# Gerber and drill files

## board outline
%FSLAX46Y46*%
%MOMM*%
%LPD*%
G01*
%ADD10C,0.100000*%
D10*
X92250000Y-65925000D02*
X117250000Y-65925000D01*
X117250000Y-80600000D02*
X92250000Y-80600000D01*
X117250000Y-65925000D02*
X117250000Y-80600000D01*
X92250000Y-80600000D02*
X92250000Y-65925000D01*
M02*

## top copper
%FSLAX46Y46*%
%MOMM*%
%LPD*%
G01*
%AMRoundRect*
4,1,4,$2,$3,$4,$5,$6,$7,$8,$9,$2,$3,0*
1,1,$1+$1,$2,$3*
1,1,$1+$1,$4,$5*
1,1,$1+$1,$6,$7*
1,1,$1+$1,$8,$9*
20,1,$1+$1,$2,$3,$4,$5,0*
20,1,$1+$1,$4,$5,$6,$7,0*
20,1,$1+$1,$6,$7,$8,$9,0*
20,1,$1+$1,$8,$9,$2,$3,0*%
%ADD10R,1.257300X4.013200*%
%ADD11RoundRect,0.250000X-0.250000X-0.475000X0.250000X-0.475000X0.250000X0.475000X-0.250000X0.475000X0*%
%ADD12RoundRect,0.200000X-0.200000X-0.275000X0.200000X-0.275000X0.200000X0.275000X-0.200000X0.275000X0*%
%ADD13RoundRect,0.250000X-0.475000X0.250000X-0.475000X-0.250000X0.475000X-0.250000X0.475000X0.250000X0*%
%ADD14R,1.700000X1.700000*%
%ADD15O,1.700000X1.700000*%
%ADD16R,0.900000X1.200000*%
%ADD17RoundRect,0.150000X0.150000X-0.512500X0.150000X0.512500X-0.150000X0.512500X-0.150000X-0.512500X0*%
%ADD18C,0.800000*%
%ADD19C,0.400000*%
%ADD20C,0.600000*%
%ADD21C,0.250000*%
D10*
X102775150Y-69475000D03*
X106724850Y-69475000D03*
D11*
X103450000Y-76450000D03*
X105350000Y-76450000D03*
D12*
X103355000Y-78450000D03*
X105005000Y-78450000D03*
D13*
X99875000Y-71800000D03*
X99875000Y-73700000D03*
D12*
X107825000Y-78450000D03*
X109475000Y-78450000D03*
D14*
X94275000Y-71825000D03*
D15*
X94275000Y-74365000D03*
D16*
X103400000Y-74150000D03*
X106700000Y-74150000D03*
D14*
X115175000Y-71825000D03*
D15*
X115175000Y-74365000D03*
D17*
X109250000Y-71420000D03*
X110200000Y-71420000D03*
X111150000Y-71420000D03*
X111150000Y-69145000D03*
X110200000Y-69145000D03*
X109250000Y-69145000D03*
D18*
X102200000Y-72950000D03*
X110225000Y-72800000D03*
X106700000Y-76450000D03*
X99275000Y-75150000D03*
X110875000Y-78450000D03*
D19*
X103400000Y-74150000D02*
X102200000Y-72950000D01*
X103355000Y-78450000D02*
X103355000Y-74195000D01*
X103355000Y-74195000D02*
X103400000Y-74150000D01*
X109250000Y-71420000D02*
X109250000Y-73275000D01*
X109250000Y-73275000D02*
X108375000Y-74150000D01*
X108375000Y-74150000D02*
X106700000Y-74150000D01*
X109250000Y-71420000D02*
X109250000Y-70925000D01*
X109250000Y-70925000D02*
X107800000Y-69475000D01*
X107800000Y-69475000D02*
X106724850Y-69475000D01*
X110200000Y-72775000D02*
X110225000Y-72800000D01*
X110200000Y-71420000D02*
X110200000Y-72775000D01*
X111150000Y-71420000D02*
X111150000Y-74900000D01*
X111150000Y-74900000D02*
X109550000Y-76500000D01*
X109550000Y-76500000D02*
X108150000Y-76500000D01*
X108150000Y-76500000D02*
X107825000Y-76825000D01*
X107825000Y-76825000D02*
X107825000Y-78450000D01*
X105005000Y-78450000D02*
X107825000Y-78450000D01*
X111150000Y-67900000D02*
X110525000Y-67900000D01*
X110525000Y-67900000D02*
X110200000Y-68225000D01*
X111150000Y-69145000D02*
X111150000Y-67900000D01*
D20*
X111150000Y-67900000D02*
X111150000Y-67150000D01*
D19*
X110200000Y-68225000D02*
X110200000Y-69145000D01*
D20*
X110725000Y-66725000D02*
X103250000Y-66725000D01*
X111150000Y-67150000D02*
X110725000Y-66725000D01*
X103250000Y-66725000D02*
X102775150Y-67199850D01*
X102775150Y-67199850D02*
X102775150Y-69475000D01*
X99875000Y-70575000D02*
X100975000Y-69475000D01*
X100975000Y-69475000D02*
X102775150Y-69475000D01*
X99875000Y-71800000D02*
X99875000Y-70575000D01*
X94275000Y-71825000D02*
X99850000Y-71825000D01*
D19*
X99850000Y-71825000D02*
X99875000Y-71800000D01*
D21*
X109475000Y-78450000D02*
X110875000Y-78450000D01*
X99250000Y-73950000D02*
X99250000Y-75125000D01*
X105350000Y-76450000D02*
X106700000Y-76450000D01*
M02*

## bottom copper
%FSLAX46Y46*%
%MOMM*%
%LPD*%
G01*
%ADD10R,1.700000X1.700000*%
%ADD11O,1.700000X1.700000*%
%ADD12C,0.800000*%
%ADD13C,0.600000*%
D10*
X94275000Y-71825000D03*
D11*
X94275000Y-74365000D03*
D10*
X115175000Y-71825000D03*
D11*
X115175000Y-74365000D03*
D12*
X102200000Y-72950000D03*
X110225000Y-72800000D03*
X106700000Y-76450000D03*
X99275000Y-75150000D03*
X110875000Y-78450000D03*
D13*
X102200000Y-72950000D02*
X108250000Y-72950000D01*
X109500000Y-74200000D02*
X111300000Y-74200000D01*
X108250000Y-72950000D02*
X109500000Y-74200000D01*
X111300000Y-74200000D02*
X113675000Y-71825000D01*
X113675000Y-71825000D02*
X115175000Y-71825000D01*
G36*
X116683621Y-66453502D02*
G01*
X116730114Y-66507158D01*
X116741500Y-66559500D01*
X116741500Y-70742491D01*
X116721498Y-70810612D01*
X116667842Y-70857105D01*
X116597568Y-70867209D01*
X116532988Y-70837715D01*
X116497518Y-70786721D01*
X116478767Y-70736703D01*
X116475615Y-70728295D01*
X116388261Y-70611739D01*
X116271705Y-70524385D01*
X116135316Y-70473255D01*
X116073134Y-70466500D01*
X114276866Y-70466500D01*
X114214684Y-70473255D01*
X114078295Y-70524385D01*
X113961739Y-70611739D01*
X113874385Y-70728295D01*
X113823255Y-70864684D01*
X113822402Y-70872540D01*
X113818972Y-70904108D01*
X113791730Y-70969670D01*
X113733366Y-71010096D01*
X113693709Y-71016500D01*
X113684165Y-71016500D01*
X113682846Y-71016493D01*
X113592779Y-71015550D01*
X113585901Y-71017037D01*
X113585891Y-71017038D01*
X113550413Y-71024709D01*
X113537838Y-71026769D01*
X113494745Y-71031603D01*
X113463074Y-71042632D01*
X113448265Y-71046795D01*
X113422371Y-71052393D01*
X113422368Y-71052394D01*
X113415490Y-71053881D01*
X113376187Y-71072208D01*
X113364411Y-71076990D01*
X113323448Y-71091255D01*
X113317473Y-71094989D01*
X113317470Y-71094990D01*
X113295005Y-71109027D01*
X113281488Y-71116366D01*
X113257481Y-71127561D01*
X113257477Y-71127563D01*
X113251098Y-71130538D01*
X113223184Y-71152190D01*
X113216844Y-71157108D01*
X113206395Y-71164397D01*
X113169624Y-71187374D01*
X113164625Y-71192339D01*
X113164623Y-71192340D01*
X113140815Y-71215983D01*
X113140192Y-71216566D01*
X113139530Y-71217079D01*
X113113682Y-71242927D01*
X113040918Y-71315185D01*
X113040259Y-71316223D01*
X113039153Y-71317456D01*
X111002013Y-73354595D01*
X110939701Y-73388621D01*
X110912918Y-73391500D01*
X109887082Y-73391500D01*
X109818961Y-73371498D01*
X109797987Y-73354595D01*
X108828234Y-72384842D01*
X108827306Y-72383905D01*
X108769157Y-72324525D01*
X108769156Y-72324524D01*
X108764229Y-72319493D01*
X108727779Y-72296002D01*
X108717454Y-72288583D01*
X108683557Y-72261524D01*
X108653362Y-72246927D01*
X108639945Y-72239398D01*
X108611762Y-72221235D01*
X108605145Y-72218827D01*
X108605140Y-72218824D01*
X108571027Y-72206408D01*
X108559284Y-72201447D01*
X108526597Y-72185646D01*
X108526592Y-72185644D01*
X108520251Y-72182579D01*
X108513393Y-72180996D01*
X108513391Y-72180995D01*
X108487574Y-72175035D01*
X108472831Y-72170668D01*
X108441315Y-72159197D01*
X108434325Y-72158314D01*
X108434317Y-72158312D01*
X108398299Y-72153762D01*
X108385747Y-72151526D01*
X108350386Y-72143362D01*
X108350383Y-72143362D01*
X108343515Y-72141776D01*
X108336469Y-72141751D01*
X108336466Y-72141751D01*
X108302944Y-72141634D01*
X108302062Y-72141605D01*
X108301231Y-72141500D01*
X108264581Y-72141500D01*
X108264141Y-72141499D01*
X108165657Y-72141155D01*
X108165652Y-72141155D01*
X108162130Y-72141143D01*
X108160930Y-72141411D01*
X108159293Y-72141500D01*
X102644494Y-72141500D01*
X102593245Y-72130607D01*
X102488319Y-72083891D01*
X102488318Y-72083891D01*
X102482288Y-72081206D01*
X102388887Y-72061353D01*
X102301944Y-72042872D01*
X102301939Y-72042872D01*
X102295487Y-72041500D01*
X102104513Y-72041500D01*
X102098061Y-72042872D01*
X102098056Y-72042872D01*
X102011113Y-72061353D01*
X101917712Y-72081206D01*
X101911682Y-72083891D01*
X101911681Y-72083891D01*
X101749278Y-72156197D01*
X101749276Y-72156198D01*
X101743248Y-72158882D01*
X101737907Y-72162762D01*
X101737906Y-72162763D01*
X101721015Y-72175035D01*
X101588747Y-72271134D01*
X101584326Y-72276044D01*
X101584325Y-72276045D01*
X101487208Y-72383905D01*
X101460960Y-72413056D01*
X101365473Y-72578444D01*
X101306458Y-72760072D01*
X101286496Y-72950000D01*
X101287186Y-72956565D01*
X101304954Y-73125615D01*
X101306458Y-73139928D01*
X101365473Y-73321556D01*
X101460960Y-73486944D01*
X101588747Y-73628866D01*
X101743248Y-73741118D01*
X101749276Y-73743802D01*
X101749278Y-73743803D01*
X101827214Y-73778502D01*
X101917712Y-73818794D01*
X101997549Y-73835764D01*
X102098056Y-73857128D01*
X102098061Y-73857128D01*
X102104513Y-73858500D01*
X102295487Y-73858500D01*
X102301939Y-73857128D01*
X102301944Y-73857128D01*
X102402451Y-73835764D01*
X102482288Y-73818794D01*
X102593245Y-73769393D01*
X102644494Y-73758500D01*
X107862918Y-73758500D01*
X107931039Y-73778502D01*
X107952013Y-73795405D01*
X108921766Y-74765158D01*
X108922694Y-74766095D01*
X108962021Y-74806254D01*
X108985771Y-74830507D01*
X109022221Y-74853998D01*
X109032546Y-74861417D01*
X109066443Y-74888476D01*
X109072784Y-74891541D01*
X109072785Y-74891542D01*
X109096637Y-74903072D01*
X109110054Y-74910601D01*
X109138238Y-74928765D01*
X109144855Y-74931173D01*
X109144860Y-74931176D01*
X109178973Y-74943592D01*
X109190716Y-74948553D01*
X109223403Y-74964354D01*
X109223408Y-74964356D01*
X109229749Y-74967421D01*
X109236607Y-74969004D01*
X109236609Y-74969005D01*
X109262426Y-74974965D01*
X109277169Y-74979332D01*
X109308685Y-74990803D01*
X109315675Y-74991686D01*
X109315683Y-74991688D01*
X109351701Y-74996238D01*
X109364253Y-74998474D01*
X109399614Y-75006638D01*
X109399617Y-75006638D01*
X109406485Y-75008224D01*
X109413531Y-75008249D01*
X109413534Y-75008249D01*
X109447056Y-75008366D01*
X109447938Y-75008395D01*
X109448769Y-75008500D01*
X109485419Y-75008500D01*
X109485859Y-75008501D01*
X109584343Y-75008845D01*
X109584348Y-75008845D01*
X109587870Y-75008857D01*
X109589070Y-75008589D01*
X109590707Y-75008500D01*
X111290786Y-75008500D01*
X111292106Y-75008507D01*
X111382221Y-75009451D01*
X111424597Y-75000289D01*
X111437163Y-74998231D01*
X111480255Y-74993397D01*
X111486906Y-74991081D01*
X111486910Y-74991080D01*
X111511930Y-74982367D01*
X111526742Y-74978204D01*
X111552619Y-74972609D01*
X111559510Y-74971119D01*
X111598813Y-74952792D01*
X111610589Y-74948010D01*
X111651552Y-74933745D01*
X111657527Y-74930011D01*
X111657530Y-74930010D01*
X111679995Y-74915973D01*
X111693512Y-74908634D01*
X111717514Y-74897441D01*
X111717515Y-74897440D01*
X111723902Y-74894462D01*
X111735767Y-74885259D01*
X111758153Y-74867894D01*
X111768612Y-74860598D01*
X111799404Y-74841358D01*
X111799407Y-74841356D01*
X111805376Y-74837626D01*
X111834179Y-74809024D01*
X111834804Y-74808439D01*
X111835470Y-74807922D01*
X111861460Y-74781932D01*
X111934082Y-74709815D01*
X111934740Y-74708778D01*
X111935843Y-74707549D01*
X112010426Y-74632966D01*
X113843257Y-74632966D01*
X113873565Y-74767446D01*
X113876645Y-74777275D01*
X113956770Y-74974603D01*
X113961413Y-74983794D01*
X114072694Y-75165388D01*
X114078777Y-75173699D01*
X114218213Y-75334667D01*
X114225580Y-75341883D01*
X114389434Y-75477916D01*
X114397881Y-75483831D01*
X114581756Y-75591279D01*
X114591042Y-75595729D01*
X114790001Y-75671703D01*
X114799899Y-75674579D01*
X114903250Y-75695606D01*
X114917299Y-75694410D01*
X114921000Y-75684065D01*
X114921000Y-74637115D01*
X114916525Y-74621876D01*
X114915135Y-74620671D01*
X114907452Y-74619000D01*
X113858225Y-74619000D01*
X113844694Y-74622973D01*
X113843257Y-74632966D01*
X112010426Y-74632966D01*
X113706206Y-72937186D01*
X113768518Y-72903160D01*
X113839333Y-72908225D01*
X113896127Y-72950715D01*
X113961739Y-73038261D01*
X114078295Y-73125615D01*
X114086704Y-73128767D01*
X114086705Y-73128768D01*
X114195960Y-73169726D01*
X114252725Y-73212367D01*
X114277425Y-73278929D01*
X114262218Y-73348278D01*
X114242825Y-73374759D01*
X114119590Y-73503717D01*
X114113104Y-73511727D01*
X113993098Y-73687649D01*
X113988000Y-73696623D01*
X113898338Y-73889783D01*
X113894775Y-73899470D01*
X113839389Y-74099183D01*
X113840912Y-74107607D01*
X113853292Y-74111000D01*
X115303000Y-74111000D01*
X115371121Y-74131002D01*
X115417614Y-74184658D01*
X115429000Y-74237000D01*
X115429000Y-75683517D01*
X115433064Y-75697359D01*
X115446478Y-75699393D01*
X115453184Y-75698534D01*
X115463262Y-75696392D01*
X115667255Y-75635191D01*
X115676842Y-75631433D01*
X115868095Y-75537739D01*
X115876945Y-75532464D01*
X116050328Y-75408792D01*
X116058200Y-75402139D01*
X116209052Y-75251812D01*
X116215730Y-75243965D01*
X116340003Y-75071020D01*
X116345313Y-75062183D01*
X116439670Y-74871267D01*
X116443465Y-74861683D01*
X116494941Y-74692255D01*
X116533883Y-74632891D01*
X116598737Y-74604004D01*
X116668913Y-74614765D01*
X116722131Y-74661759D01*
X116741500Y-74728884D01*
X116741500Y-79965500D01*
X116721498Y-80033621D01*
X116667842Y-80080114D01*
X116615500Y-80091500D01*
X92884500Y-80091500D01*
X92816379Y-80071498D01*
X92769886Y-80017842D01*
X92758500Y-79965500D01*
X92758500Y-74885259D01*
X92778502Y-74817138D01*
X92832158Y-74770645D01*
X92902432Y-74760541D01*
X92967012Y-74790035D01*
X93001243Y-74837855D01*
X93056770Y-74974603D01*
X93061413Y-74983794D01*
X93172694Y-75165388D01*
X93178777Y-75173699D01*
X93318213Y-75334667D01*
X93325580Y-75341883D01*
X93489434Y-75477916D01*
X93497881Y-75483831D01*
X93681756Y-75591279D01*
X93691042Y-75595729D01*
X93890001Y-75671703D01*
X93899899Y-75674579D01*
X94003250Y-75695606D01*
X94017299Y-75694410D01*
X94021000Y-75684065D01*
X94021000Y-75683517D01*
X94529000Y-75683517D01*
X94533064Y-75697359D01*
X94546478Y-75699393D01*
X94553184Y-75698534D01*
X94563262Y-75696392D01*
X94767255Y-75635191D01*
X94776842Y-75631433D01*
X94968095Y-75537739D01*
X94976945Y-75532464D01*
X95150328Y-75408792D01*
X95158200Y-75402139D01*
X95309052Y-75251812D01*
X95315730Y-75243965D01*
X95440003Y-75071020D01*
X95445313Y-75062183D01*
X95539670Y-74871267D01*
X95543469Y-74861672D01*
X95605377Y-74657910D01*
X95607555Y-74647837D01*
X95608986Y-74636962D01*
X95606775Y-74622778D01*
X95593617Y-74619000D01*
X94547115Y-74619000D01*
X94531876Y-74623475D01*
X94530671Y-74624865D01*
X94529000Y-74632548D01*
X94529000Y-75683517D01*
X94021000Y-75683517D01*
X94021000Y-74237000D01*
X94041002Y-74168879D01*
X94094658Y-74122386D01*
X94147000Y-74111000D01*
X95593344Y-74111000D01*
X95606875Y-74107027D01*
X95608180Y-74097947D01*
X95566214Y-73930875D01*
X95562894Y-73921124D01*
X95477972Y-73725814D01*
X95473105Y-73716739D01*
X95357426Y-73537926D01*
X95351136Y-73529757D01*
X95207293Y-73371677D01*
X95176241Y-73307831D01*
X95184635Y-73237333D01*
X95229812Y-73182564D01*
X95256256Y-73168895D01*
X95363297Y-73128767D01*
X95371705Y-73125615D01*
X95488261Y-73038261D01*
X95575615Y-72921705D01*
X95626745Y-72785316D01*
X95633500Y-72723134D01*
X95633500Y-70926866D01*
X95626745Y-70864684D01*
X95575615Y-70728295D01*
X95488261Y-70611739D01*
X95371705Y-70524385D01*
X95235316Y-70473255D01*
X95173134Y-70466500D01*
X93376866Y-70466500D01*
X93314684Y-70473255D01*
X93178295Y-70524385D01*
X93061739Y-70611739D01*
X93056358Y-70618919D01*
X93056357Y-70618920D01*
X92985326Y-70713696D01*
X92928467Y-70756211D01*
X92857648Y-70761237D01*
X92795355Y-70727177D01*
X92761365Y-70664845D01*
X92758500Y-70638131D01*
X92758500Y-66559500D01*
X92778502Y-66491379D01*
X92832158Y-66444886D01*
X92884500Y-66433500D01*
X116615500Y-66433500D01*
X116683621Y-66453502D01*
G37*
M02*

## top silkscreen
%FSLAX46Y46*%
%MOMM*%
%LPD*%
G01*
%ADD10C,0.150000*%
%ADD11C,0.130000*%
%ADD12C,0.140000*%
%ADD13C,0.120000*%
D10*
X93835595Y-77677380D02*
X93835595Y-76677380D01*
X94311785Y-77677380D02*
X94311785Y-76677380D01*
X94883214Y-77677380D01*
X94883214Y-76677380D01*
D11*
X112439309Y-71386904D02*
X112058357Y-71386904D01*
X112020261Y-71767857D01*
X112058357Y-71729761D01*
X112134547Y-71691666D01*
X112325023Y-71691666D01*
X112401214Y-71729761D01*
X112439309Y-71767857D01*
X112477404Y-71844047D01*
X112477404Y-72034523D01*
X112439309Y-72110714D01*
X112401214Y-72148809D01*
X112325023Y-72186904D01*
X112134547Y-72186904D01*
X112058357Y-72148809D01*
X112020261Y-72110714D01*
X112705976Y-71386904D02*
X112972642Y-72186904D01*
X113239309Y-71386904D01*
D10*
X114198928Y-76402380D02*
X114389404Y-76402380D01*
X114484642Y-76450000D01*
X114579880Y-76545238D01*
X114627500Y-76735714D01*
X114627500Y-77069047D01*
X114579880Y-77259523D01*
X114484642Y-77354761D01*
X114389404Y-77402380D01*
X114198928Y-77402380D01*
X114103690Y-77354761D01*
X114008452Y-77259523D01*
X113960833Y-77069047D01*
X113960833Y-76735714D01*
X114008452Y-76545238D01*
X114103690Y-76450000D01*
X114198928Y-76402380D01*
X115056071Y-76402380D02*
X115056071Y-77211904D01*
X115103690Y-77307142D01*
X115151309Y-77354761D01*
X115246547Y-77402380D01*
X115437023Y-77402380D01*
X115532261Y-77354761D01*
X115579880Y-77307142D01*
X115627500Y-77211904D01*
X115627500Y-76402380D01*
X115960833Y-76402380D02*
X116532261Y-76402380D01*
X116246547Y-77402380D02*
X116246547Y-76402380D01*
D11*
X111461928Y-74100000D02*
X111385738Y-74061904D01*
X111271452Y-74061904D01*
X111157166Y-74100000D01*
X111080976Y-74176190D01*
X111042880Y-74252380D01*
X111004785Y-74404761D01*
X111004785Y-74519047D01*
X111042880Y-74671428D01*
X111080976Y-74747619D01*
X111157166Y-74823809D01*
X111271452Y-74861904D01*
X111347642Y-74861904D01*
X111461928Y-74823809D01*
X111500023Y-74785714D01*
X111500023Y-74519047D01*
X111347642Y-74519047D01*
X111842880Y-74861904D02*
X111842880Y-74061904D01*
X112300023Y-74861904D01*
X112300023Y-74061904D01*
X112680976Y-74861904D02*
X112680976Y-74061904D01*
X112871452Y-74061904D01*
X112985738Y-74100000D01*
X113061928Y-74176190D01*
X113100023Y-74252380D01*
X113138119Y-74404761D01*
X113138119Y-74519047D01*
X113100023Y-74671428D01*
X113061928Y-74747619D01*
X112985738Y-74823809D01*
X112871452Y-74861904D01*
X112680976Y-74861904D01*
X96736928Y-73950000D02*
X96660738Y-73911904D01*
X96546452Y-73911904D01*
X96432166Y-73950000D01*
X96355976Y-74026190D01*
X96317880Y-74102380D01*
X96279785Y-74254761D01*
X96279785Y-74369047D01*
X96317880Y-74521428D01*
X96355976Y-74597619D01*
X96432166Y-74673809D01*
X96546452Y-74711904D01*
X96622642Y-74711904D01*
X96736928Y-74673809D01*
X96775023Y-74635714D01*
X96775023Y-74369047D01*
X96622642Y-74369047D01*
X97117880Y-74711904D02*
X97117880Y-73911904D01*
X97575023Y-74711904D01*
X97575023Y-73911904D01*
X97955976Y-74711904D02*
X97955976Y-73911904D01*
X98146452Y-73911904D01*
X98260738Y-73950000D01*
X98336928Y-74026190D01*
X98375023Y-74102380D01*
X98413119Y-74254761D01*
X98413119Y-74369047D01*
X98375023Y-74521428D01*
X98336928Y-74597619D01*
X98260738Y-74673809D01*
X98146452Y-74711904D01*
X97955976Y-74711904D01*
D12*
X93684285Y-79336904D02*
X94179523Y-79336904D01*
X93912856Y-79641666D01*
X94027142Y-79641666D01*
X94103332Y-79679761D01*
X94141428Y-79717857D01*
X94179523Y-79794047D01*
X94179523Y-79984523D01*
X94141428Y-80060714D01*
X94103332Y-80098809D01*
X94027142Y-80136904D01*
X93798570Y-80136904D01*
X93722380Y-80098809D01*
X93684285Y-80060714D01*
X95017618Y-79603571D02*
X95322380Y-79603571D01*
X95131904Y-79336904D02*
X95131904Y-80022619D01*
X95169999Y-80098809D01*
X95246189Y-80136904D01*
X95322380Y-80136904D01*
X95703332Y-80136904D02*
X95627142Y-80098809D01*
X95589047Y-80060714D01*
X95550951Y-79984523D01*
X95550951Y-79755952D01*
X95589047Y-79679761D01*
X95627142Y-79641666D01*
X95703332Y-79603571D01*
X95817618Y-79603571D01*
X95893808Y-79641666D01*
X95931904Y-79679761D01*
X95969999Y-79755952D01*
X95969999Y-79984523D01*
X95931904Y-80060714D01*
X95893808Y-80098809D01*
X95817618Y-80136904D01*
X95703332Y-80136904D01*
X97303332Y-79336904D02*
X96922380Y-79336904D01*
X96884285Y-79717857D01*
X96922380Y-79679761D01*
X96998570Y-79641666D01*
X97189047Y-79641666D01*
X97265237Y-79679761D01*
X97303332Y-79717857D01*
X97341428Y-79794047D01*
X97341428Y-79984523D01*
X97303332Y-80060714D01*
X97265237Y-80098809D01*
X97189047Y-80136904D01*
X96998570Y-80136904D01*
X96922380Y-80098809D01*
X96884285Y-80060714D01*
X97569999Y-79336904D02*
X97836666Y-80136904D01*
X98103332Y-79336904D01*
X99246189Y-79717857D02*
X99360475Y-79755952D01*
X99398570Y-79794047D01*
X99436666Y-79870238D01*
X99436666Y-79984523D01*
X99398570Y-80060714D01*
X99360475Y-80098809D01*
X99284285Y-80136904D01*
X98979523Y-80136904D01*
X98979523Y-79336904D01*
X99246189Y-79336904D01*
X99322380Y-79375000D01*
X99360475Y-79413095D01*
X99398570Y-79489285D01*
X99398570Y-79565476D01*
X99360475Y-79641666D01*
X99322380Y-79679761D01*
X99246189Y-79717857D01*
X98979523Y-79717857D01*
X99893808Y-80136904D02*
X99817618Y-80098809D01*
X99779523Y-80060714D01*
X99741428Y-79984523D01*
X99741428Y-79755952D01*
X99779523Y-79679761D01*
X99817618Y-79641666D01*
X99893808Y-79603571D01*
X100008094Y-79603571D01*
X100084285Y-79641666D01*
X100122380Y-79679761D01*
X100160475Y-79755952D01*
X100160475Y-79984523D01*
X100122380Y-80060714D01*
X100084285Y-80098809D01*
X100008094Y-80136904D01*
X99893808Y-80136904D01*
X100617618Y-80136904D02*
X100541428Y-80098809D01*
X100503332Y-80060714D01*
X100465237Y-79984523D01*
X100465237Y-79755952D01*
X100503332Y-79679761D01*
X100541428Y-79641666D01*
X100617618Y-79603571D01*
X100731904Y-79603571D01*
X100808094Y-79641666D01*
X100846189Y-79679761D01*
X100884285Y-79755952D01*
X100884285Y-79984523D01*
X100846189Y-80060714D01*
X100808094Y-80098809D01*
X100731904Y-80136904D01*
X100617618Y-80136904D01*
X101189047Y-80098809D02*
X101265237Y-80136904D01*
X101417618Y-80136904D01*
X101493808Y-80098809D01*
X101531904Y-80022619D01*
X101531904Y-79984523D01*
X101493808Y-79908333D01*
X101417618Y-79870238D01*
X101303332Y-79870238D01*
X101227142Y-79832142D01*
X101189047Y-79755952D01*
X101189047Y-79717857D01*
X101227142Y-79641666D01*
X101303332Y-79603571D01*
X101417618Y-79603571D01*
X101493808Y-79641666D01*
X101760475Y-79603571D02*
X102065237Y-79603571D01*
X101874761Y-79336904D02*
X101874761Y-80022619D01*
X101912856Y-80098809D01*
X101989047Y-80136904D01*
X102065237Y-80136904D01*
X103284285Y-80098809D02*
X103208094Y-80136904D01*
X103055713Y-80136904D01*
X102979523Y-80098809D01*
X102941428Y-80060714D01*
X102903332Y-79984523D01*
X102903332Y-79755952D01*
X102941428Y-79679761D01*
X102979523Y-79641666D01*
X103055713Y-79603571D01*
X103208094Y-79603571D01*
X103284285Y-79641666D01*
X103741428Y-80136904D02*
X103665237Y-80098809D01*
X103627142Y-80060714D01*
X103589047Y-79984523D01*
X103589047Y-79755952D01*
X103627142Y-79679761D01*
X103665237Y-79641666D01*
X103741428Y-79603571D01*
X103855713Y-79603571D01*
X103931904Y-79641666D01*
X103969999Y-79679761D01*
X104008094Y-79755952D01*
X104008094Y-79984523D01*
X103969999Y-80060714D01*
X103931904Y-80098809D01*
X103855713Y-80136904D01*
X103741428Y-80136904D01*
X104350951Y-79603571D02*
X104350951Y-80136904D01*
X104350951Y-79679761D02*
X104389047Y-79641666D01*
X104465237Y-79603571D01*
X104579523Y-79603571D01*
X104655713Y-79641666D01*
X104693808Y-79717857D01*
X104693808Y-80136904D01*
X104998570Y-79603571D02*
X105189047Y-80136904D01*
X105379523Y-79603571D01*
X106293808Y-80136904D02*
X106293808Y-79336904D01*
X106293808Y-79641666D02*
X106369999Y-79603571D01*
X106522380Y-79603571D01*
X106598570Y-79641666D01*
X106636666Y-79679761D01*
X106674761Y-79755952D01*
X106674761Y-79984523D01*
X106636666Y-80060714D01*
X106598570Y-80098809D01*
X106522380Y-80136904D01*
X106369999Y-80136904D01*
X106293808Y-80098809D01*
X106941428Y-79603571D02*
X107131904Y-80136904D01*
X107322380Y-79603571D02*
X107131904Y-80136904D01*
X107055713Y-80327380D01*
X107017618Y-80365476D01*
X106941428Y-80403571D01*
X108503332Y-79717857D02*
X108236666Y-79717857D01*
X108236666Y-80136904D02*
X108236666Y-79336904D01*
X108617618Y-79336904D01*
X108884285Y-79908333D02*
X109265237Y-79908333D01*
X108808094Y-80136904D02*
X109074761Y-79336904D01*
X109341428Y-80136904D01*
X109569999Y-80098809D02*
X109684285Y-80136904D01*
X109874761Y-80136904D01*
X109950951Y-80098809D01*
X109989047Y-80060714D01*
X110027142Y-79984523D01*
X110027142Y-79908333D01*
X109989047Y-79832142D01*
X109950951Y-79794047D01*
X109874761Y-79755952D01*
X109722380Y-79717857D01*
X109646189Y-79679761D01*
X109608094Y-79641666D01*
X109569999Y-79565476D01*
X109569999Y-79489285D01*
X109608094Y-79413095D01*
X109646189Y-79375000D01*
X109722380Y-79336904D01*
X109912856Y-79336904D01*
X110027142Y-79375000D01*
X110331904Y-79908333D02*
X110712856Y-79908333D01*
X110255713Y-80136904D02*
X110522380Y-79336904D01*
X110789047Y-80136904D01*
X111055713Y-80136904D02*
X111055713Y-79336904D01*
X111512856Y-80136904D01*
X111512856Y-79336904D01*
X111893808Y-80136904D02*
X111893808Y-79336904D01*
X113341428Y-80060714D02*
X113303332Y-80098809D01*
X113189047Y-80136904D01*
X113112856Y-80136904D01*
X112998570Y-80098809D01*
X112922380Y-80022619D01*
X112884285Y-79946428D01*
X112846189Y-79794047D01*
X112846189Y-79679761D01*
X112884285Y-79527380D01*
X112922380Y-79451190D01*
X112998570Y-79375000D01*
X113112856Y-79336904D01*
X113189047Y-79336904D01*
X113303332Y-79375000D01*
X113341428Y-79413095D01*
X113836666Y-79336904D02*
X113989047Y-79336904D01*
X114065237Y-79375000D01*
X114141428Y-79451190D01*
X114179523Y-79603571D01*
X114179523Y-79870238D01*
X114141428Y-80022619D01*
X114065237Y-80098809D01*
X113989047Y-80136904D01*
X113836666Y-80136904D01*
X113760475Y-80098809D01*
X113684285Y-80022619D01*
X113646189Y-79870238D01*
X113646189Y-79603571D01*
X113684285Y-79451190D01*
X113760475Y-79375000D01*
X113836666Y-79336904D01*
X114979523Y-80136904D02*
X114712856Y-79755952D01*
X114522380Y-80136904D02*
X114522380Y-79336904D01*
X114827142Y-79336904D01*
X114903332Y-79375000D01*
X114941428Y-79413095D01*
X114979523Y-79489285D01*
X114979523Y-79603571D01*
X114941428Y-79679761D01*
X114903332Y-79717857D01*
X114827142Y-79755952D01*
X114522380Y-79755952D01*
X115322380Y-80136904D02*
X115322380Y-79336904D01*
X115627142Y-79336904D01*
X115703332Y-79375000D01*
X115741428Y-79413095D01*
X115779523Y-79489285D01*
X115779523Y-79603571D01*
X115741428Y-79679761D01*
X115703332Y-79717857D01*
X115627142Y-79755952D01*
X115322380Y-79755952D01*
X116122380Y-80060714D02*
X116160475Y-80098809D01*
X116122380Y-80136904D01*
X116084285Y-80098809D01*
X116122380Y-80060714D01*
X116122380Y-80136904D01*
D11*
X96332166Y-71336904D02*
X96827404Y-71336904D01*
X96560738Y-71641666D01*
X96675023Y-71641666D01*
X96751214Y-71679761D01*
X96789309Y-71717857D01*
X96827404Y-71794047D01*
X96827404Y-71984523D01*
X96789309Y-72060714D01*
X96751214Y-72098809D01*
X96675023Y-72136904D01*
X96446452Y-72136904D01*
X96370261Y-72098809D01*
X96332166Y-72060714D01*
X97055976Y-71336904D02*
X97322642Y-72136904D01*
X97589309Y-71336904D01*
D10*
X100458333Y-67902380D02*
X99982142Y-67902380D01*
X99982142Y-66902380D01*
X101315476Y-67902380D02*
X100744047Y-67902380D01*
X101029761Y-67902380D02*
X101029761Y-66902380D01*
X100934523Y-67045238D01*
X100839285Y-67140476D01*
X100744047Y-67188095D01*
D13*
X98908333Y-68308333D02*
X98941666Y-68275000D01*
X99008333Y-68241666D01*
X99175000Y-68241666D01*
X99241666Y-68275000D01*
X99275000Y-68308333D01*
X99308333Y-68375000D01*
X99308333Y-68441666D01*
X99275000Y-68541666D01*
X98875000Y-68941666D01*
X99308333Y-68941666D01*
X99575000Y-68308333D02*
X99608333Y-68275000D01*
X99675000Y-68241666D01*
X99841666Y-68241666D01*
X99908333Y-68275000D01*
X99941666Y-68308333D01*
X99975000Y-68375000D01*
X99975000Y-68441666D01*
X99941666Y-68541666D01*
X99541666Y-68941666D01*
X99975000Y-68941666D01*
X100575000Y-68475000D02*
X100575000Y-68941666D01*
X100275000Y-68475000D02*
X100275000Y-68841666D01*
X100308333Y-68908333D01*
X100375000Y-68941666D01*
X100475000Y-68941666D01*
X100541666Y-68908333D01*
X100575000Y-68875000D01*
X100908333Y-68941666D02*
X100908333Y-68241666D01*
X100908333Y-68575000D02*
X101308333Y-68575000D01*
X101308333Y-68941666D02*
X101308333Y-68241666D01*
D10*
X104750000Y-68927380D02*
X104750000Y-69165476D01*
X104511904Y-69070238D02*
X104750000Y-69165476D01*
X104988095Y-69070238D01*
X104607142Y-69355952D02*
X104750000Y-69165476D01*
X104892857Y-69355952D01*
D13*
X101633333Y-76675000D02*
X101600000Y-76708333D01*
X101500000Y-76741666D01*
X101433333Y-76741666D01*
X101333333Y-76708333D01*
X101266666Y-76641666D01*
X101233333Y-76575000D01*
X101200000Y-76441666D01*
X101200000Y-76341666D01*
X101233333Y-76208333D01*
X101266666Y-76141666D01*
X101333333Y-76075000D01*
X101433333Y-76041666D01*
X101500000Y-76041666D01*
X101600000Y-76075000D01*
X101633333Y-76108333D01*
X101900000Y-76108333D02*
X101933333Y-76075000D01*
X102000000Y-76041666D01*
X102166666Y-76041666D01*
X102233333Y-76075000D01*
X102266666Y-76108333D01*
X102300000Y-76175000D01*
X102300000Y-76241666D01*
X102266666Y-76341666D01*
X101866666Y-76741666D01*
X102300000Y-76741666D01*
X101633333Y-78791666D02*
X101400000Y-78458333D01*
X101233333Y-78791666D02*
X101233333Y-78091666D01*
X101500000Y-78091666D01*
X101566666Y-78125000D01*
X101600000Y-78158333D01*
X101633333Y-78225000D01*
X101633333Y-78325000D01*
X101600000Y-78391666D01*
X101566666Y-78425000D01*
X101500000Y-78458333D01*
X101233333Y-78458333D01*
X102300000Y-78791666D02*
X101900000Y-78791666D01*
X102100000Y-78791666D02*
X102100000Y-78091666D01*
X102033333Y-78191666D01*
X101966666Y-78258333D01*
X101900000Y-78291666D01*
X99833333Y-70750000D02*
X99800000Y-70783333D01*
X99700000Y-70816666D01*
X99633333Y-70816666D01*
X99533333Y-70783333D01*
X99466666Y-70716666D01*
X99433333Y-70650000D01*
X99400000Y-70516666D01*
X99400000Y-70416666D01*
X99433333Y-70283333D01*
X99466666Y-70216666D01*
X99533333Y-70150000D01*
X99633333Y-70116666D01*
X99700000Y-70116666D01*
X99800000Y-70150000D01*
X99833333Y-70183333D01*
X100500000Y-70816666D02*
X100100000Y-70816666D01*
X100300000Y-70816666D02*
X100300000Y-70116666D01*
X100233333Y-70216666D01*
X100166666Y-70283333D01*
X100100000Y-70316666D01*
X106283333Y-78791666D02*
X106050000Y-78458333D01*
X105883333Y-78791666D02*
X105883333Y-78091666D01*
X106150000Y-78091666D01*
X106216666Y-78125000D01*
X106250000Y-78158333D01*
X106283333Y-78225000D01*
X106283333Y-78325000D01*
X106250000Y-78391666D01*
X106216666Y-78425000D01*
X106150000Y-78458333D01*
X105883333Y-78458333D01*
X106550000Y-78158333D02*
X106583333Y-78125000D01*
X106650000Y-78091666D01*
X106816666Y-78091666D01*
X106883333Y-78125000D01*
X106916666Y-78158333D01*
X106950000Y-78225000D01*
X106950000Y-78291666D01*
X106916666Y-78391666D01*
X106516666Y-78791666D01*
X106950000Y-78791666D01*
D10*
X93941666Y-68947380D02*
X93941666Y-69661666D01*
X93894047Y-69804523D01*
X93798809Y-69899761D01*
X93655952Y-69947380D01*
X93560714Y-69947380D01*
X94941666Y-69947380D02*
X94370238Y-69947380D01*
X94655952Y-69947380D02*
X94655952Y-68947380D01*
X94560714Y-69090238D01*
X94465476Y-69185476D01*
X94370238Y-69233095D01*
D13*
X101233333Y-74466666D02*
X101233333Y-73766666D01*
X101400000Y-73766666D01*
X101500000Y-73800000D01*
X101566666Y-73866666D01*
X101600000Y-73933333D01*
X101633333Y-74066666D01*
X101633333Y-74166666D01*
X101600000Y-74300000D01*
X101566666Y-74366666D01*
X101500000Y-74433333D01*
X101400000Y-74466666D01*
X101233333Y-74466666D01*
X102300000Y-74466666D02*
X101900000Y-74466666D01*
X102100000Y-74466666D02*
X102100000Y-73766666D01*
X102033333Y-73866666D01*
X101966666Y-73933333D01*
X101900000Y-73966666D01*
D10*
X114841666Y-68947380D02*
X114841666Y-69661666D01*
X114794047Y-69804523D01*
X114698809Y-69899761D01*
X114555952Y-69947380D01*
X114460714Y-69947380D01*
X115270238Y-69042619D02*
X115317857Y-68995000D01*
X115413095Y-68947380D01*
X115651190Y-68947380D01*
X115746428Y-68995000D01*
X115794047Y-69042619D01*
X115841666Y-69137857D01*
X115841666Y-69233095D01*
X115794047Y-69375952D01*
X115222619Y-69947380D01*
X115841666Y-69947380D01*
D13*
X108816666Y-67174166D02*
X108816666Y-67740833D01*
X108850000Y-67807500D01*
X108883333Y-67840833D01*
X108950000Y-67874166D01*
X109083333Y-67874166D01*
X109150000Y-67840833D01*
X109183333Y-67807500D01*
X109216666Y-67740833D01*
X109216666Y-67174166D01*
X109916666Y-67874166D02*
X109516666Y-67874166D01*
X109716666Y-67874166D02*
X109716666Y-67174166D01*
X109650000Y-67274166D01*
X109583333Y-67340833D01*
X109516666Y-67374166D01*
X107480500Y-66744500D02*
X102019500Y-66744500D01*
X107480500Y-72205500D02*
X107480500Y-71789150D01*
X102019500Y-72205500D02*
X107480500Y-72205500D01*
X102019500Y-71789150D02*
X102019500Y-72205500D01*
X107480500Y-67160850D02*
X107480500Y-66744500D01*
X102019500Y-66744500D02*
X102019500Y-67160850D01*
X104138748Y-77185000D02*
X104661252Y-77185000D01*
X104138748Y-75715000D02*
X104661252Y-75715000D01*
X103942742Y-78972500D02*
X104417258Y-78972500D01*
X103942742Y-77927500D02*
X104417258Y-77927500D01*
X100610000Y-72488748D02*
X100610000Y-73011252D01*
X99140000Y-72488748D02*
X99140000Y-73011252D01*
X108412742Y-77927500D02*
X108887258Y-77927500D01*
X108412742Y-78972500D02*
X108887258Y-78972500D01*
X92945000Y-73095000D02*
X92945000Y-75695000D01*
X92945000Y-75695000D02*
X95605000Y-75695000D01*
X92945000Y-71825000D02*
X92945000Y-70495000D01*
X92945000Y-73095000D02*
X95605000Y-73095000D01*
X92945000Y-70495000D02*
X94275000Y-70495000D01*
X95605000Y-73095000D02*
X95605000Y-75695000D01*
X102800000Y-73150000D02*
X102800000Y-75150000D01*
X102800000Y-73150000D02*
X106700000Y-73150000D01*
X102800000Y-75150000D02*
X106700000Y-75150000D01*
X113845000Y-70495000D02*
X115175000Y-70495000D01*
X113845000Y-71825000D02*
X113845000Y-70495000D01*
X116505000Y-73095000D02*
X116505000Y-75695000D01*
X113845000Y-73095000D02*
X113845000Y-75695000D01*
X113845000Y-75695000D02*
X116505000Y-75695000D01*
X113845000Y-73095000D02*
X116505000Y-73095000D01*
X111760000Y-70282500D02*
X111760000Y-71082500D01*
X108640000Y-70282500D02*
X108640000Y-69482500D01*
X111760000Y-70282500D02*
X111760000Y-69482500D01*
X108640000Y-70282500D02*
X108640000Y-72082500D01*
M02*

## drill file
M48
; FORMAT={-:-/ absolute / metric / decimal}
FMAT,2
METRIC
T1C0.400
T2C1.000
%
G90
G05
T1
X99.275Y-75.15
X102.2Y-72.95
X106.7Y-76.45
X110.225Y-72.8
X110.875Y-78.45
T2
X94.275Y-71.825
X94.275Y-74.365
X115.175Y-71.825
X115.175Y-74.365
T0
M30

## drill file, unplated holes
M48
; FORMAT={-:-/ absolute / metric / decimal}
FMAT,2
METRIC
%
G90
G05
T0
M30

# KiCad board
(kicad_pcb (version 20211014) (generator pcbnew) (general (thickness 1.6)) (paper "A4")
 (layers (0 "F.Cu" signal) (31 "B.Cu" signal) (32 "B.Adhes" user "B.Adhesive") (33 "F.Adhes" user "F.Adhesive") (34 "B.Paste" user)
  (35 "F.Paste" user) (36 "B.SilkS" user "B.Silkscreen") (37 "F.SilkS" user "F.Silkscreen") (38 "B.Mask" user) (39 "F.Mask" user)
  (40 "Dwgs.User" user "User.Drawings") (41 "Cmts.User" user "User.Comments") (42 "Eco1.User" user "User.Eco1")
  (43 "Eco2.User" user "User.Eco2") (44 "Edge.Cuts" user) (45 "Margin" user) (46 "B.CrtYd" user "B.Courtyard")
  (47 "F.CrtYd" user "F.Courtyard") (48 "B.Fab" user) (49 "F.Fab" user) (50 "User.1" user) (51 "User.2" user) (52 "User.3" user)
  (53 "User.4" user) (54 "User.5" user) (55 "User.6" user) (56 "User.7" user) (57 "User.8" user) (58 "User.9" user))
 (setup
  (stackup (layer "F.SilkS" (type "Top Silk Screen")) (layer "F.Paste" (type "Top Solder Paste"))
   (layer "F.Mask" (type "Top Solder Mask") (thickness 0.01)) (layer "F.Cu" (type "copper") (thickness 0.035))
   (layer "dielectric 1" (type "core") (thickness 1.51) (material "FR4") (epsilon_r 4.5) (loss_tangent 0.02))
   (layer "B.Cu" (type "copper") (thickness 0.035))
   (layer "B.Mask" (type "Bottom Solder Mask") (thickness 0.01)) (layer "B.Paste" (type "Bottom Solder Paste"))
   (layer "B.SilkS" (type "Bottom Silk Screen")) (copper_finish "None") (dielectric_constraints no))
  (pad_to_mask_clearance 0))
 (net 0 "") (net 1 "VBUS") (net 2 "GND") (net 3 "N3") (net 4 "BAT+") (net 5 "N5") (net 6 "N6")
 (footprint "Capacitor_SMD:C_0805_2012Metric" (layer "F.Cu") (at 104.4 76.45)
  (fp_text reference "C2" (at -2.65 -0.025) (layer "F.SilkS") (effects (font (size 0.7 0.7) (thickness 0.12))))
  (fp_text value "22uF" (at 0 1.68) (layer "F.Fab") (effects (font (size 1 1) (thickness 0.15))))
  (fp_line (start -0.261252 0.735) (end 0.261252 0.735) (layer "F.SilkS") (width 0.12))
  (fp_line (start -0.261252 -0.735) (end 0.261252 -0.735) (layer "F.SilkS") (width 0.12))
  (pad "1" smd roundrect (at -0.95 0) (size 1 1.45) (layers "F.Cu" "F.Paste" "F.Mask") (roundrect_rratio 0.25) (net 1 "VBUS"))
  (pad "2" smd roundrect (at 0.95 0) (size 1 1.45) (layers "F.Cu" "F.Paste" "F.Mask") (roundrect_rratio 0.25) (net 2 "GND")))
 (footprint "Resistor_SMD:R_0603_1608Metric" (layer "F.Cu") (at 104.18 78.45)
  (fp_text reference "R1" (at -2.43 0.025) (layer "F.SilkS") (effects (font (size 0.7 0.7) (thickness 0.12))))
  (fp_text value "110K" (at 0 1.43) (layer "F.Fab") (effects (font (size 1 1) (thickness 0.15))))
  (fp_line (start -0.237258 0.5225) (end 0.237258 0.5225) (layer "F.SilkS") (width 0.12))
  (fp_line (start -0.237258 -0.5225) (end 0.237258 -0.5225) (layer "F.SilkS") (width 0.12))
  (pad "1" smd roundrect (at -0.825 0) (size 0.8 0.95) (layers "F.Cu" "F.Paste" "F.Mask") (roundrect_rratio 0.25) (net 1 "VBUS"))
  (pad "2" smd roundrect (at 0.825 0) (size 0.8 0.95) (layers "F.Cu" "F.Paste" "F.Mask") (roundrect_rratio 0.25) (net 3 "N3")))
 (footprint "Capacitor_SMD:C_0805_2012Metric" (layer "F.Cu") (at 99.875 72.75 -90)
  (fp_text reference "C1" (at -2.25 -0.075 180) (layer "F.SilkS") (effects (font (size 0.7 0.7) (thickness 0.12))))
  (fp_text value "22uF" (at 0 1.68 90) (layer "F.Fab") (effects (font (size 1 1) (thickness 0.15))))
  (fp_line (start -0.261252 -0.735) (end 0.261252 -0.735) (layer "F.SilkS") (width 0.12))
  (fp_line (start -0.261252 0.735) (end 0.261252 0.735) (layer "F.SilkS") (width 0.12))
  (pad "1" smd roundrect (at -0.95 0 270) (size 1 1.45) (layers "F.Cu" "F.Paste" "F.Mask") (roundrect_rratio 0.25) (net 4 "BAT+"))
  (pad "2" smd roundrect (at 0.95 0 270) (size 1 1.45) (layers "F.Cu" "F.Paste" "F.Mask") (roundrect_rratio 0.25) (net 2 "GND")))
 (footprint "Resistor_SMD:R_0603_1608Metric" (layer "F.Cu") (at 108.65 78.45)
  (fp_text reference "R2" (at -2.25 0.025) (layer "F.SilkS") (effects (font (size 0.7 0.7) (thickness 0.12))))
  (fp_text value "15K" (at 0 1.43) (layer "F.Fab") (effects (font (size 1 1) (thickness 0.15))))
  (fp_line (start -0.237258 -0.5225) (end 0.237258 -0.5225) (layer "F.SilkS") (width 0.12))
  (fp_line (start -0.237258 0.5225) (end 0.237258 0.5225) (layer "F.SilkS") (width 0.12))
  (pad "1" smd roundrect (at -0.825 0) (size 0.8 0.95) (layers "F.Cu" "F.Paste" "F.Mask") (roundrect_rratio 0.25) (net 3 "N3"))
  (pad "2" smd roundrect (at 0.825 0) (size 0.8 0.95) (layers "F.Cu" "F.Paste" "F.Mask") (roundrect_rratio 0.25) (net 2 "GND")))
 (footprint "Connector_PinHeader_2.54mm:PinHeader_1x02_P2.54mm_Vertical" (layer "F.Cu") (at 94.275 71.825)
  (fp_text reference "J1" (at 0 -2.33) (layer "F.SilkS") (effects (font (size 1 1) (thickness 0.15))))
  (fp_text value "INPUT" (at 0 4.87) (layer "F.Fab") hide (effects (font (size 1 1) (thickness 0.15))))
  (fp_line (start -1.33 1.27) (end -1.33 3.87) (layer "F.SilkS") (width 0.12))
  (fp_line (start -1.33 3.87) (end 1.33 3.87) (layer "F.SilkS") (width 0.12))
  (fp_line (start -1.33 0) (end -1.33 -1.33) (layer "F.SilkS") (width 0.12))
  (fp_line (start -1.33 1.27) (end 1.33 1.27) (layer "F.SilkS") (width 0.12))
  (fp_line (start -1.33 -1.33) (end 0 -1.33) (layer "F.SilkS") (width 0.12))
  (fp_line (start 1.33 1.27) (end 1.33 3.87) (layer "F.SilkS") (width 0.12))
  (pad "1" thru_hole rect (at 0 0) (size 1.7 1.7) (drill 1) (layers *.Cu *.Mask) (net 4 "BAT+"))
  (pad "2" thru_hole oval (at 0 2.54) (size 1.7 1.7) (drill 1) (layers *.Cu *.Mask) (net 2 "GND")))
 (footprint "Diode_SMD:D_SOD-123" (layer "F.Cu") (at 105.05 74.15)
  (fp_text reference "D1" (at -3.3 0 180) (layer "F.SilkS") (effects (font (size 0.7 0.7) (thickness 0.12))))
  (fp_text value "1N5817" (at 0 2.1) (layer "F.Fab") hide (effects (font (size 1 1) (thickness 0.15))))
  (fp_line (start -2.25 -1) (end -2.25 1) (layer "F.SilkS") (width 0.12))
  (fp_line (start -2.25 -1) (end 1.65 -1) (layer "F.SilkS") (width 0.12))
  (fp_line (start -2.25 1) (end 1.65 1) (layer "F.SilkS") (width 0.12))
  (pad "1" smd rect (at -1.65 0) (size 0.9 1.2) (layers "F.Cu" "F.Paste" "F.Mask") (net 1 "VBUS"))
  (pad "2" smd rect (at 1.65 0) (size 0.9 1.2) (layers "F.Cu" "F.Paste" "F.Mask") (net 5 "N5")))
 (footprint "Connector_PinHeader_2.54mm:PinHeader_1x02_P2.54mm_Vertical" (layer "F.Cu") (at 115.175 71.825)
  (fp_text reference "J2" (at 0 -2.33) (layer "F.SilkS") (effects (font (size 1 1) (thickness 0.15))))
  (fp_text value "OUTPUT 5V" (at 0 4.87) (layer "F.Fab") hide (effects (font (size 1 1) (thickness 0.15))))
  (fp_line (start -1.33 -1.33) (end 0 -1.33) (layer "F.SilkS") (width 0.12))
  (fp_line (start -1.33 0) (end -1.33 -1.33) (layer "F.SilkS") (width 0.12))
  (fp_line (start 1.33 1.27) (end 1.33 3.87) (layer "F.SilkS") (width 0.12))
  (fp_line (start -1.33 1.27) (end -1.33 3.87) (layer "F.SilkS") (width 0.12))
  (fp_line (start -1.33 3.87) (end 1.33 3.87) (layer "F.SilkS") (width 0.12))
  (fp_line (start -1.33 1.27) (end 1.33 1.27) (layer "F.SilkS") (width 0.12))
  (pad "1" thru_hole rect (at 0 0) (size 1.7 1.7) (drill 1) (layers *.Cu *.Mask) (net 1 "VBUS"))
  (pad "2" thru_hole oval (at 0 2.54) (size 1.7 1.7) (drill 1) (layers *.Cu *.Mask) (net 2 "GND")))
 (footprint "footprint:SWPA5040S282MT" (layer "F.Cu") (at 104.75 69.475)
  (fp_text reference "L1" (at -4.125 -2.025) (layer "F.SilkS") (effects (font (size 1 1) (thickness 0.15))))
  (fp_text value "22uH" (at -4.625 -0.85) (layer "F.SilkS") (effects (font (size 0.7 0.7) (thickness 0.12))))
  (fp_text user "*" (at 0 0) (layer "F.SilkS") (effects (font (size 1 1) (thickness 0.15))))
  (fp_line (start 2.7305 -2.31415) (end 2.7305 -2.7305) (layer "F.SilkS") (width 0.12))
  (fp_line (start 2.7305 2.7305) (end 2.7305 2.31415) (layer "F.SilkS") (width 0.12))
  (fp_line (start -2.7305 -2.7305) (end -2.7305 -2.31415) (layer "F.SilkS") (width 0.12))
  (fp_line (start -2.7305 2.31415) (end -2.7305 2.7305) (layer "F.SilkS") (width 0.12))
  (fp_line (start -2.7305 2.7305) (end 2.7305 2.7305) (layer "F.SilkS") (width 0.12))
  (fp_line (start 2.7305 -2.7305) (end -2.7305 -2.7305) (layer "F.SilkS") (width 0.12))
  (pad "1" smd rect (at -1.97485 0) (size 1.2573 4.0132) (layers "F.Cu" "F.Paste" "F.Mask") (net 4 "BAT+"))
  (pad "2" smd rect (at 1.97485 0) (size 1.2573 4.0132) (layers "F.Cu" "F.Paste" "F.Mask") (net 5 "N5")))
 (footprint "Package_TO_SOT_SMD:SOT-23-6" (layer "F.Cu") (at 110.2 70.2825 90)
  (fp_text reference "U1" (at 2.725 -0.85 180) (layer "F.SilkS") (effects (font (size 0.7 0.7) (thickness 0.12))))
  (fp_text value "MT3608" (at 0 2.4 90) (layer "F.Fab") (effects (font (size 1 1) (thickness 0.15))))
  (fp_line (start 0 1.56) (end -0.8 1.56) (layer "F.SilkS") (width 0.12))
  (fp_line (start 0 -1.56) (end 0.8 -1.56) (layer "F.SilkS") (width 0.12))
  (fp_line (start 0 1.56) (end 0.8 1.56) (layer "F.SilkS") (width 0.12))
  (fp_line (start 0 -1.56) (end -1.8 -1.56) (layer "F.SilkS") (width 0.12))
  (pad "1" smd roundrect (at -1.1375 -0.95 90) (size 1.325 0.6) (layers "F.Cu" "F.Paste" "F.Mask") (roundrect_rratio 0.25) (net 5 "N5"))
  (pad "2" smd roundrect (at -1.1375 0 90) (size 1.325 0.6) (layers "F.Cu" "F.Paste" "F.Mask") (roundrect_rratio 0.25) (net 2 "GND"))
  (pad "3" smd roundrect (at -1.1375 0.95 90) (size 1.325 0.6) (layers "F.Cu" "F.Paste" "F.Mask") (roundrect_rratio 0.25) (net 3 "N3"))
  (pad "4" smd roundrect (at 1.1375 0.95 90) (size 1.325 0.6) (layers "F.Cu" "F.Paste" "F.Mask") (roundrect_rratio 0.25) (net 4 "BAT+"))
  (pad "5" smd roundrect (at 1.1375 0 90) (size 1.325 0.6) (layers "F.Cu" "F.Paste" "F.Mask") (roundrect_rratio 0.25) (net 4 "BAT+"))
  (pad "6" smd roundrect (at 1.1375 -0.95 90) (size 1.325 0.6) (layers "F.Cu" "F.Paste" "F.Mask") (roundrect_rratio 0.25) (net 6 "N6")))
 (gr_line (start 92.25 65.925) (end 117.25 65.925) (layer "Edge.Cuts") (width 0.1))
 (gr_line (start 117.25 80.6) (end 92.25 80.6) (layer "Edge.Cuts") (width 0.1))
 (gr_line (start 117.25 65.925) (end 117.25 80.6) (layer "Edge.Cuts") (width 0.1))
 (gr_line (start 92.25 80.6) (end 92.25 65.925) (layer "Edge.Cuts") (width 0.1))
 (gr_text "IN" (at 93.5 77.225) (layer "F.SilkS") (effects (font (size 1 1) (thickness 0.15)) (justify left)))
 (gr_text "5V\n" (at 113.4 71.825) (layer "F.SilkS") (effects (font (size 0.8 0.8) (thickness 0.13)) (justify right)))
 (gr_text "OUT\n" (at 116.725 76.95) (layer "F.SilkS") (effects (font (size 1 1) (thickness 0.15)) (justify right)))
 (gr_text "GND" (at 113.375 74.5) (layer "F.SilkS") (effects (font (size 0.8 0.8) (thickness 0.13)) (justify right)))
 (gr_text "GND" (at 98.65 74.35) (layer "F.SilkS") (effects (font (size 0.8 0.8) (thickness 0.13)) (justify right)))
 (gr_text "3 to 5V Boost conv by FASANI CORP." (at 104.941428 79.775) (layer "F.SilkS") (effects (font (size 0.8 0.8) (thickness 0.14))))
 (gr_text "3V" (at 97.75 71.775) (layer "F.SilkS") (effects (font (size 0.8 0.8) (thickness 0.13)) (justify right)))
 (segment (start 102.77515 67.19985) (end 102.77515 69.475) (width 0.6) (layer "F.Cu") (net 4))
 (segment (start 111.15 67.9) (end 111.15 67.15) (width 0.6) (layer "F.Cu") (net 4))
 (segment (start 103.25 66.725) (end 102.77515 67.19985) (width 0.6) (layer "F.Cu") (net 4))
 (segment (start 99.85 71.825) (end 99.875 71.8) (width 0.4) (layer "F.Cu") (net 4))
 (segment (start 99.875 70.575) (end 100.975 69.475) (width 0.6) (layer "F.Cu") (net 4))
 (segment (start 110.525 67.9) (end 110.2 68.225) (width 0.4) (layer "F.Cu") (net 4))
 (segment (start 110.725 66.725) (end 103.25 66.725) (width 0.6) (layer "F.Cu") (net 4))
 (segment (start 111.15 67.9) (end 110.525 67.9) (width 0.4) (layer "F.Cu") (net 4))
 (segment (start 99.875 71.8) (end 99.875 70.575) (width 0.6) (layer "F.Cu") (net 4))
 (segment (start 111.15 69.145) (end 111.15 67.9) (width 0.4) (layer "F.Cu") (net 4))
 (segment (start 110.2 68.225) (end 110.2 69.145) (width 0.4) (layer "F.Cu") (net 4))
 (segment (start 94.275 71.825) (end 99.85 71.825) (width 0.6) (layer "F.Cu") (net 4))
 (segment (start 100.975 69.475) (end 102.77515 69.475) (width 0.6) (layer "F.Cu") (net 4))
 (segment (start 111.15 67.15) (end 110.725 66.725) (width 0.6) (layer "F.Cu") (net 4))
 (segment (start 109.25 71.42) (end 109.25 73.275) (width 0.4) (layer "F.Cu") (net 5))
 (segment (start 107.8 69.475) (end 106.72485 69.475) (width 0.4) (layer "F.Cu") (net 5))
 (segment (start 108.375 74.15) (end 106.7 74.15) (width 0.4) (layer "F.Cu") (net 5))
 (segment (start 109.25 73.275) (end 108.375 74.15) (width 0.4) (layer "F.Cu") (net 5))
 (segment (start 109.25 70.925) (end 107.8 69.475) (width 0.4) (layer "F.Cu") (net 5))
 (segment (start 109.25 71.42) (end 109.25 70.925) (width 0.4) (layer "F.Cu") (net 5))
 (segment (start 103.4 74.15) (end 102.2 72.95) (width 0.4) (layer "F.Cu") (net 1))
 (segment (start 103.355 78.45) (end 103.355 74.195) (width 0.4) (layer "F.Cu") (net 1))
 (segment (start 103.355 74.195) (end 103.4 74.15) (width 0.4) (layer "F.Cu") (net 1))
 (via (at 102.2 72.95) (size 0.8) (drill 0.4) (layers "F.Cu" "B.Cu") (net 1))
 (segment (start 113.675 71.825) (end 115.175 71.825) (width 0.6) (layer "B.Cu") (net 1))
 (segment (start 108.25 72.95) (end 109.5 74.2) (width 0.6) (layer "B.Cu") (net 1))
 (segment (start 109.5 74.2) (end 111.3 74.2) (width 0.6) (layer "B.Cu") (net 1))
 (segment (start 102.2 72.95) (end 108.25 72.95) (width 0.6) (layer "B.Cu") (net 1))
 (segment (start 111.3 74.2) (end 113.675 71.825) (width 0.6) (layer "B.Cu") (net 1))
 (segment (start 111.15 74.9) (end 109.55 76.5) (width 0.4) (layer "F.Cu") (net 3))
 (segment (start 111.15 71.42) (end 111.15 74.9) (width 0.4) (layer "F.Cu") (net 3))
 (segment (start 105.005 78.45) (end 107.825 78.45) (width 0.4) (layer "F.Cu") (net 3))
 (segment (start 108.15 76.5) (end 107.825 76.825) (width 0.4) (layer "F.Cu") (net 3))
 (segment (start 107.825 76.825) (end 107.825 78.45) (width 0.4) (layer "F.Cu") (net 3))
 (segment (start 109.55 76.5) (end 108.15 76.5) (width 0.4) (layer "F.Cu") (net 3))
 (segment (start 109.475 78.45) (end 110.875 78.45) (width 0.25) (layer "F.Cu") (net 2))
 (segment (start 99.25 73.95) (end 99.25 75.125) (width 0.25) (layer "F.Cu") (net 2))
 (segment (start 110.2 71.42) (end 110.2 72.775) (width 0.4) (layer "F.Cu") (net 2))
 (segment (start 105.35 76.45) (end 106.7 76.45) (width 0.25) (layer "F.Cu") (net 2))
 (segment (start 110.2 72.775) (end 110.225 72.8) (width 0.4) (layer "F.Cu") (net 2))
 (via (at 110.225 72.8) (size 0.8) (drill 0.4) (layers "F.Cu" "B.Cu") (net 2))
 (via (at 106.7 76.45) (size 0.8) (drill 0.4) (layers "F.Cu" "B.Cu") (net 2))
 (via (at 99.275 75.15) (size 0.8) (drill 0.4) (layers "F.Cu" "B.Cu") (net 2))
 (via (at 110.875 78.45) (size 0.8) (drill 0.4) (layers "F.Cu" "B.Cu") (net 2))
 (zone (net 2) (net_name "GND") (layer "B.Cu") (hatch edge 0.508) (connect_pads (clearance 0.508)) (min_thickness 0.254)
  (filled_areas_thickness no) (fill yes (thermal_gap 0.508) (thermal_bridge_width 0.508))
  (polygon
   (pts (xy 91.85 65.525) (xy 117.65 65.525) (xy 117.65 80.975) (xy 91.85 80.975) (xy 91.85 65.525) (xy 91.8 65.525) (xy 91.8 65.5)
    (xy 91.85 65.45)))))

